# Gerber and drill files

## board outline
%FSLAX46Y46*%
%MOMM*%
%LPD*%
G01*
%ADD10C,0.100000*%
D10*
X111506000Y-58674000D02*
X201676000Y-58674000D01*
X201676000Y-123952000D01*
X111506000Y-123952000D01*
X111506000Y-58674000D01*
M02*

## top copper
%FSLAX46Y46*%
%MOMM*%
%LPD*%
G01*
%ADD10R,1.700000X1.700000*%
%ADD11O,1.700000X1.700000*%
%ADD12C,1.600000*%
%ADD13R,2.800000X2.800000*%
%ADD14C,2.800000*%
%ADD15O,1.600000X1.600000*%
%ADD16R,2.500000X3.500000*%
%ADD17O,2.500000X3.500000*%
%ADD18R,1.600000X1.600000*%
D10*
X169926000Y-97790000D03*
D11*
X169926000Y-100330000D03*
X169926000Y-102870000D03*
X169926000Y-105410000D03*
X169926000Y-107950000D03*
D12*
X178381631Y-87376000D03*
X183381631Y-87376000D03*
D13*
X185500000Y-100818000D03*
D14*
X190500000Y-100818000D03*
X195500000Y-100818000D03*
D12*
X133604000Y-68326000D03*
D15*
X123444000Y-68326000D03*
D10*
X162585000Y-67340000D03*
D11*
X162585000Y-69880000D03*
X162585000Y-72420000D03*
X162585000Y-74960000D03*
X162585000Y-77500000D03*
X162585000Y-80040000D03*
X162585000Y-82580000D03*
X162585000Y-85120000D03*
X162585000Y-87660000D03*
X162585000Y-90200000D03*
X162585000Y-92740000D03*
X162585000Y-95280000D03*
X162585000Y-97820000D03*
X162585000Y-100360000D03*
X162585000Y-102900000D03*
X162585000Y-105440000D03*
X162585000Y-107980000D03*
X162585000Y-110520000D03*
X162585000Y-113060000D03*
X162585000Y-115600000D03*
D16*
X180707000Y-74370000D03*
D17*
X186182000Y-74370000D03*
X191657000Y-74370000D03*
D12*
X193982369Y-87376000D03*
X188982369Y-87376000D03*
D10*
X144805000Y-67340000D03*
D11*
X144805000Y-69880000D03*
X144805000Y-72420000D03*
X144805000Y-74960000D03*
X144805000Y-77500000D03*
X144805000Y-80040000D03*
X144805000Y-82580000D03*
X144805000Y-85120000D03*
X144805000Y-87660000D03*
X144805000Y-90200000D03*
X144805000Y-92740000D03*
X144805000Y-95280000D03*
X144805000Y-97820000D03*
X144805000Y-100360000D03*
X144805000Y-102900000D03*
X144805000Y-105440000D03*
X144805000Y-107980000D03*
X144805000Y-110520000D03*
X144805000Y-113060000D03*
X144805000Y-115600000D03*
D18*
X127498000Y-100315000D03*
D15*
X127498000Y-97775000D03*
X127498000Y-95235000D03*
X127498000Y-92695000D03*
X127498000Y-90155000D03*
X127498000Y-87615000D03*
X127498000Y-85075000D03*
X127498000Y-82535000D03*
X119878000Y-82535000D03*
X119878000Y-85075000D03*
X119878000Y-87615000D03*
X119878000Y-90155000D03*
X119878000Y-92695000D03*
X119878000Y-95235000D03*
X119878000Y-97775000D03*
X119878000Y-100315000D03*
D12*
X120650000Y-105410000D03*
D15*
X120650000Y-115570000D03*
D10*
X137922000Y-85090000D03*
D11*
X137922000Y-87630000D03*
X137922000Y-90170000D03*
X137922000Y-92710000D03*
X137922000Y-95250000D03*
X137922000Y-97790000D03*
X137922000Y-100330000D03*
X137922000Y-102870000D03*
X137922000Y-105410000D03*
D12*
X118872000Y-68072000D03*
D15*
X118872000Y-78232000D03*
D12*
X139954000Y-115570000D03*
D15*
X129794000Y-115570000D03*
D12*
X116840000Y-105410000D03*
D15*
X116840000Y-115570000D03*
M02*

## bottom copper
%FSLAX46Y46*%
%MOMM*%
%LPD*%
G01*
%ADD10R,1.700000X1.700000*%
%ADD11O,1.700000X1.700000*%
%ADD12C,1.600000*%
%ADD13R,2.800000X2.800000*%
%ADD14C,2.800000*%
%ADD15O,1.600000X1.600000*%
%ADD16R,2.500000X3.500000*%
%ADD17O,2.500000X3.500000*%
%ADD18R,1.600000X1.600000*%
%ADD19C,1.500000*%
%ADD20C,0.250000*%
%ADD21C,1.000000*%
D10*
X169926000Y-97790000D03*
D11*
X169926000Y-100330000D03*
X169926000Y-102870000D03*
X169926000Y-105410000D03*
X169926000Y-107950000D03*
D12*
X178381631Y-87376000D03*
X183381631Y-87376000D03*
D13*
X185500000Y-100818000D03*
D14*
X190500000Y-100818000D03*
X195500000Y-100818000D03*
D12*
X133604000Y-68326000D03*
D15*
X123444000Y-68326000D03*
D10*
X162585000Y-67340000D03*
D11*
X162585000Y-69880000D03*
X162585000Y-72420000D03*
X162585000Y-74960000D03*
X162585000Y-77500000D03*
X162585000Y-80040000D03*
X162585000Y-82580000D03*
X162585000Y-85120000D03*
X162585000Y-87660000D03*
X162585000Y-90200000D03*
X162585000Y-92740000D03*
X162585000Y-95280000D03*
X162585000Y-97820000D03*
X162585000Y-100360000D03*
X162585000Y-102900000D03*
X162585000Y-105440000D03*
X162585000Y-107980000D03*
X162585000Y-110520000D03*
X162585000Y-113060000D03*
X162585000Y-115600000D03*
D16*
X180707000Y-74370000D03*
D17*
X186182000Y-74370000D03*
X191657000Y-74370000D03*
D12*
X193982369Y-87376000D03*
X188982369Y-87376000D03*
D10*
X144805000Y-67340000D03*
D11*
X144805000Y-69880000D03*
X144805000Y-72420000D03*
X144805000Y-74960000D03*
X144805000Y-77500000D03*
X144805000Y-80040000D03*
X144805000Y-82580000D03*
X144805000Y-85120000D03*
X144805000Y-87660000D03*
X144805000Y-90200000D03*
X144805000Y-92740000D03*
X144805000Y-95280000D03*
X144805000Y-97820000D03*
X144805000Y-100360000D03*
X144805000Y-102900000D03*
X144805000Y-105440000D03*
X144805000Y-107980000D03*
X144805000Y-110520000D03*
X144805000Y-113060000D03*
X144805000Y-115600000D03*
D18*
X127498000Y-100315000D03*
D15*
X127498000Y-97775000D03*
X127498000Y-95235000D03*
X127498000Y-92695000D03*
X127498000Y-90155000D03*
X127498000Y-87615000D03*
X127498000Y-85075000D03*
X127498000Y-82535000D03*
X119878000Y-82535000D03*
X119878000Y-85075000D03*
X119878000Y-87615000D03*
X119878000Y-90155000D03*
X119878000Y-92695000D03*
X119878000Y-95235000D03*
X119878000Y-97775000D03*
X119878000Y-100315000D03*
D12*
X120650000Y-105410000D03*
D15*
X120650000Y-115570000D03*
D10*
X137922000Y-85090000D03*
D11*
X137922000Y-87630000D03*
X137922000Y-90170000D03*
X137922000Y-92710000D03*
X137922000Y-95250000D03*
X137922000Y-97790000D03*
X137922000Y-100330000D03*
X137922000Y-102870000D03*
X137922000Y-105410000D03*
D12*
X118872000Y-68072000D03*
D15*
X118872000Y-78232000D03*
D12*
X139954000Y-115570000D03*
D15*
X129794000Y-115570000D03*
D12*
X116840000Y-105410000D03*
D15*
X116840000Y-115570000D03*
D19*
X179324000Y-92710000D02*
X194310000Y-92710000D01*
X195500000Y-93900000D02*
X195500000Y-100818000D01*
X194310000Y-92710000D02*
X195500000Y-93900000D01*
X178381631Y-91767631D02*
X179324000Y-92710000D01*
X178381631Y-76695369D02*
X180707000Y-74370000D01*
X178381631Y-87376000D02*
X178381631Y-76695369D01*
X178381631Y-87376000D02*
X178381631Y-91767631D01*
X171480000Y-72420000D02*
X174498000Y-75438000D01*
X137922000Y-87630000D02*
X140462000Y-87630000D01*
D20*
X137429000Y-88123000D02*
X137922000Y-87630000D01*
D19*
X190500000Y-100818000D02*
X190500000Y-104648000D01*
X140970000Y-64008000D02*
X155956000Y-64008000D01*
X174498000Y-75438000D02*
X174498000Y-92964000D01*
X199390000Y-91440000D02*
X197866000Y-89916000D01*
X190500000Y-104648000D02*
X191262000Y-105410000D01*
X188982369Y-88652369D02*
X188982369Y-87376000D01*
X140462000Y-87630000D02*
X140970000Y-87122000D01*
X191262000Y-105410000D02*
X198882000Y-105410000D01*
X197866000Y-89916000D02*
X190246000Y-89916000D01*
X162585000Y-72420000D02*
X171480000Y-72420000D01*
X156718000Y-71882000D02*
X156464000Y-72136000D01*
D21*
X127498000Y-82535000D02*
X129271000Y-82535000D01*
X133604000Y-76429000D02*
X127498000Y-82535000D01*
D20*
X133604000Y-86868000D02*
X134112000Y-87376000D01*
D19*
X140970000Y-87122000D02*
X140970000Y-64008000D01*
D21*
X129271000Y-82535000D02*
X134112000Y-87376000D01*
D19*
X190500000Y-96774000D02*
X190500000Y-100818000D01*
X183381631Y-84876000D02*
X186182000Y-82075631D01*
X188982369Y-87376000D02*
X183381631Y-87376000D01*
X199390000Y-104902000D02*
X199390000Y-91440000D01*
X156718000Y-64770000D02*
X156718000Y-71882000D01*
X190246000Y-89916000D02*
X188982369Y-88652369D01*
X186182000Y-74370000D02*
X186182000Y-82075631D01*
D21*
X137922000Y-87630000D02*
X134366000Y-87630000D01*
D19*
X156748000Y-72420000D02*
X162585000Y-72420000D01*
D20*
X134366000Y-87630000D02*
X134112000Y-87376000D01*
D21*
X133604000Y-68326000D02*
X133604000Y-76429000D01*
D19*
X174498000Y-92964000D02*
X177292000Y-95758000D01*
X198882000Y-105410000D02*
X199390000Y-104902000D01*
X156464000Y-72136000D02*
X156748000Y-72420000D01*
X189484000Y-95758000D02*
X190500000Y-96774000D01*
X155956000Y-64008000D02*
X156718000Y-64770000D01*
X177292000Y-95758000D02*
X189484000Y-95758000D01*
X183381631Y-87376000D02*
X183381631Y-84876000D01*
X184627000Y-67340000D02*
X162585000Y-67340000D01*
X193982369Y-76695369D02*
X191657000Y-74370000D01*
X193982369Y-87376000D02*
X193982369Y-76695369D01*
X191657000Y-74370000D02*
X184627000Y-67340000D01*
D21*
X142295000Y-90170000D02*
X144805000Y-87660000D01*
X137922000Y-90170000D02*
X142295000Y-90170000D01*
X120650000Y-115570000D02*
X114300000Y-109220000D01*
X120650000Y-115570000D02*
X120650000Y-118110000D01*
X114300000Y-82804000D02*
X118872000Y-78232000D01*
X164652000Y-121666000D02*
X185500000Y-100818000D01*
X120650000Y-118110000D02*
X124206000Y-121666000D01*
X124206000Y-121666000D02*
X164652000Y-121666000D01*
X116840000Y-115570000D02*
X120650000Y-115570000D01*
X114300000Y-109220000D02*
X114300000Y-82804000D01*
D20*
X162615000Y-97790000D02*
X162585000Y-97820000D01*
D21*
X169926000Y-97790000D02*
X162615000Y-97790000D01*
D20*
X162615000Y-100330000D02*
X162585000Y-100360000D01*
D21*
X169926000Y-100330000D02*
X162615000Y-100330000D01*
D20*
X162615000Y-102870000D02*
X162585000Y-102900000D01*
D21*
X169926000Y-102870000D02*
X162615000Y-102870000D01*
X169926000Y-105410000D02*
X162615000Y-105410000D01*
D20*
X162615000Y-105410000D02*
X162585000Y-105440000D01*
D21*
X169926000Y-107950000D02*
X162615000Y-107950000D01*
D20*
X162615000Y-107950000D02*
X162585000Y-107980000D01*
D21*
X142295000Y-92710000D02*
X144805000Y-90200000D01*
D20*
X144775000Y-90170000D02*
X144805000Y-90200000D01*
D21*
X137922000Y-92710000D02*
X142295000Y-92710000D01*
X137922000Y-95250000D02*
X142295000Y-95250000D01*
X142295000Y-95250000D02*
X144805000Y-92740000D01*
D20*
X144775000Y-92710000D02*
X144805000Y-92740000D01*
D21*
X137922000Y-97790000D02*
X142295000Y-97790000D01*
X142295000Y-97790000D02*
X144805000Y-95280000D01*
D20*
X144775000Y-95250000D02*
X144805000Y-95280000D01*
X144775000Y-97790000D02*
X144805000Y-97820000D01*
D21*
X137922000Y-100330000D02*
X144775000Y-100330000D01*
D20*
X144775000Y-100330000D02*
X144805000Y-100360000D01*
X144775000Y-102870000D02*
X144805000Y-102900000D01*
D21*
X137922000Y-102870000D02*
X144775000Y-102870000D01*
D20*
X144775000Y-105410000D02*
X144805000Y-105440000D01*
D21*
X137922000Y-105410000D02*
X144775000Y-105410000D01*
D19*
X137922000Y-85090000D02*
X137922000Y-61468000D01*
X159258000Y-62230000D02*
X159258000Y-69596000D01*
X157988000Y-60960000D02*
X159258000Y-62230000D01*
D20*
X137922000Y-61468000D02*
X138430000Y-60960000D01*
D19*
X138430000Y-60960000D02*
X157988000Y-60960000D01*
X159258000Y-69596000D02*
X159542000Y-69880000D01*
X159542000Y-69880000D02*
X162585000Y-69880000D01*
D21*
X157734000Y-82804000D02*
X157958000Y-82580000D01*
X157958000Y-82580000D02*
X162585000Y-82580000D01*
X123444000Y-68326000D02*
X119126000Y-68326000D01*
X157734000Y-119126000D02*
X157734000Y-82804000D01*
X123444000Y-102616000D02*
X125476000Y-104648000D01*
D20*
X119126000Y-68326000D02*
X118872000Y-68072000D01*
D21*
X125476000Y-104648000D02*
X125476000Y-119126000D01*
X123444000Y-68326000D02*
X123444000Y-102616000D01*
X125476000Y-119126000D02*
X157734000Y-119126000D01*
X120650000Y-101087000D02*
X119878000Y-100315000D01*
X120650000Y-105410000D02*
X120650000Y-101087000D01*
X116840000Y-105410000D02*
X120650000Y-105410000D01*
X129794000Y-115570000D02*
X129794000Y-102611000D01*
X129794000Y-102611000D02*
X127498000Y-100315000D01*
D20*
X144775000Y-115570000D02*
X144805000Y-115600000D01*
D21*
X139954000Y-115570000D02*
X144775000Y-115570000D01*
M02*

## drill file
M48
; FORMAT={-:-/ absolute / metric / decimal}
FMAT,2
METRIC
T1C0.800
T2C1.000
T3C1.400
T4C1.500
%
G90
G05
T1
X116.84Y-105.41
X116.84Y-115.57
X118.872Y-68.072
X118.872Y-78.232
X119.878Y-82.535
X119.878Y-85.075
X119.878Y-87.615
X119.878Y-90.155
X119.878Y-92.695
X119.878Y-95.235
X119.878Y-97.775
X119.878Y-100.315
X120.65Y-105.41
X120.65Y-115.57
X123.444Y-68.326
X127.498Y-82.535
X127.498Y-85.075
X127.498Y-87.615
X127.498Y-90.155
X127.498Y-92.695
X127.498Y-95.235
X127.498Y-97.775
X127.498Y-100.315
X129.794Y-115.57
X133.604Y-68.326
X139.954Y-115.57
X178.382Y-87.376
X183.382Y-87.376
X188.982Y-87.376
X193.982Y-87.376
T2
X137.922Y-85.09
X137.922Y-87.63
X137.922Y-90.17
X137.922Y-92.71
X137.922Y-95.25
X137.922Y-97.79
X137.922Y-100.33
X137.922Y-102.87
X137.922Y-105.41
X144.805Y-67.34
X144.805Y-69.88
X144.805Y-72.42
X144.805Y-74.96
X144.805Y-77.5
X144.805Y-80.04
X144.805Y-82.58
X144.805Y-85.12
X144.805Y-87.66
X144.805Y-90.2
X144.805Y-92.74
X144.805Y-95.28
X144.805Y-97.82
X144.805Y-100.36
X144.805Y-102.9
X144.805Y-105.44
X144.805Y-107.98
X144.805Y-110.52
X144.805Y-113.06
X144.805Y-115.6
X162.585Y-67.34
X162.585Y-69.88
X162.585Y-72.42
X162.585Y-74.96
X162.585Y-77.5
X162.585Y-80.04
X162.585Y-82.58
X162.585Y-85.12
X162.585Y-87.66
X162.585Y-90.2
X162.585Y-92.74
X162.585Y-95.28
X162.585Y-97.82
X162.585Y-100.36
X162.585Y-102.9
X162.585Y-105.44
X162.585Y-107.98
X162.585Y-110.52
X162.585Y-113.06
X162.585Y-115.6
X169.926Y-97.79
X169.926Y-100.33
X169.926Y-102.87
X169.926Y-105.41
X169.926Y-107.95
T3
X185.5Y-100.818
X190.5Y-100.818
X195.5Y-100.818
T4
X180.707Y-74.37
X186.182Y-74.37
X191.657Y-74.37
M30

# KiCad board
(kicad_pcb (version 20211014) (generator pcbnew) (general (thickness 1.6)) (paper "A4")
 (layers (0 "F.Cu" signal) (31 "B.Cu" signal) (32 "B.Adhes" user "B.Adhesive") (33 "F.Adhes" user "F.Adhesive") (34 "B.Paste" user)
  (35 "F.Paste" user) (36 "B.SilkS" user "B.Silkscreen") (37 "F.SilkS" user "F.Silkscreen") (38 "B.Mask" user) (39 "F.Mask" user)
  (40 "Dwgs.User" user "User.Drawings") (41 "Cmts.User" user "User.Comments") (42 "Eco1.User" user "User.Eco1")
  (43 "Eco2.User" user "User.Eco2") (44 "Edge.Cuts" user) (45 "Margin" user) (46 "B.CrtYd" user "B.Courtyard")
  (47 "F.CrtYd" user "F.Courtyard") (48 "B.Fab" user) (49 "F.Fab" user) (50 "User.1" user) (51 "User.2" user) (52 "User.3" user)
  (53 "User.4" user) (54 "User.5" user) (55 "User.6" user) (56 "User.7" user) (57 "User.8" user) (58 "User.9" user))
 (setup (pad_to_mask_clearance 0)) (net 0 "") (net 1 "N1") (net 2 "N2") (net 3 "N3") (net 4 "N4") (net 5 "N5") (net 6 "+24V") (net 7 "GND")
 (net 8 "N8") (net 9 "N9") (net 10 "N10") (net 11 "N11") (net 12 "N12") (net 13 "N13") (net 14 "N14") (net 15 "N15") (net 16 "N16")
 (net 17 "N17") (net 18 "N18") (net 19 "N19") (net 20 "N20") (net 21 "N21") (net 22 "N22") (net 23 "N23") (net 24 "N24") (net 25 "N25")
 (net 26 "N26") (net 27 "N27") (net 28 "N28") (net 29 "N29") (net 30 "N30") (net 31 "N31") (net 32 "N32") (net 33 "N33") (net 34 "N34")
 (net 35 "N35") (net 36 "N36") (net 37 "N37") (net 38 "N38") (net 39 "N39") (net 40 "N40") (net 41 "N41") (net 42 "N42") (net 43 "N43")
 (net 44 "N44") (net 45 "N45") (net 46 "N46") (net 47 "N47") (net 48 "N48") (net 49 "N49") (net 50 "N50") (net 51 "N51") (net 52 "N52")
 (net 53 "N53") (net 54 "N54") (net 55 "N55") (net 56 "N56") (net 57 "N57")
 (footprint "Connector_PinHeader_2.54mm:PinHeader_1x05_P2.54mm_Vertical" (layer "F.Cu") (at 169.926 97.79)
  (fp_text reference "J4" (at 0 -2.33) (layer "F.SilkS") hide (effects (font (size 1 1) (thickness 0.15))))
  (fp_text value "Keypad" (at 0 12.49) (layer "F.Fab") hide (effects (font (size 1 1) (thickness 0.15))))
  (pad "1" thru_hole rect (at 0 0) (size 1.7 1.7) (drill 1) (layers *.Cu *.Mask) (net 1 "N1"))
  (pad "2" thru_hole oval (at 0 2.54) (size 1.7 1.7) (drill 1) (layers *.Cu *.Mask) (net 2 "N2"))
  (pad "3" thru_hole oval (at 0 5.08) (size 1.7 1.7) (drill 1) (layers *.Cu *.Mask) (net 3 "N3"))
  (pad "4" thru_hole oval (at 0 7.62) (size 1.7 1.7) (drill 1) (layers *.Cu *.Mask) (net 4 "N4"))
  (pad "5" thru_hole oval (at 0 10.16) (size 1.7 1.7) (drill 1) (layers *.Cu *.Mask) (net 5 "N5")))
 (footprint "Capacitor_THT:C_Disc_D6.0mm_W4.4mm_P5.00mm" (layer "F.Cu") (at 178.381631 87.376)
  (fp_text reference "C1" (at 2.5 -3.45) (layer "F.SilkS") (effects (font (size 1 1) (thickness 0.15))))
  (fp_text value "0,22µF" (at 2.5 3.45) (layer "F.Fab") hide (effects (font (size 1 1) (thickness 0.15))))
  (pad "1" thru_hole circle (at 0 0) (size 1.6 1.6) (drill 0.8) (layers *.Cu *.Mask) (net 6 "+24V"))
  (pad "2" thru_hole circle (at 5 0) (size 1.6 1.6) (drill 0.8) (layers *.Cu *.Mask) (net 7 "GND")))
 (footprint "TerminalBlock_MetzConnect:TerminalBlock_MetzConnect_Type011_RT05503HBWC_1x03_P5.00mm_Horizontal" (layer "F.Cu")
  (at 185.5 100.818)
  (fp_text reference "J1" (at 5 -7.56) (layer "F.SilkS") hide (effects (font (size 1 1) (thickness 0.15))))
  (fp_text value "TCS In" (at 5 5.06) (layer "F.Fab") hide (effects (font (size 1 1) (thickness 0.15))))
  (pad "1" thru_hole rect (at 0 0) (size 2.8 2.8) (drill 1.4) (layers *.Cu *.Mask) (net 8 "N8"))
  (pad "2" thru_hole circle (at 5 0) (size 2.8 2.8) (drill 1.4) (layers *.Cu *.Mask) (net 7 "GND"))
  (pad "3" thru_hole circle (at 10 0) (size 2.8 2.8) (drill 1.4) (layers *.Cu *.Mask) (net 6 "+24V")))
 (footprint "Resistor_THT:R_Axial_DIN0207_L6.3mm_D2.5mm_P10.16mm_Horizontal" (layer "F.Cu") (at 133.604 68.326 180)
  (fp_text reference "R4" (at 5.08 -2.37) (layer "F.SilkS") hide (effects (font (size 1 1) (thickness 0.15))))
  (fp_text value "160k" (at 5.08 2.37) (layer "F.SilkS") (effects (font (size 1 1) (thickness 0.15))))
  (pad "1" thru_hole circle (at 0 0 180) (size 1.6 1.6) (drill 0.8) (layers *.Cu *.Mask) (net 7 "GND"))
  (pad "2" thru_hole oval (at 10.16 0 180) (size 1.6 1.6) (drill 0.8) (layers *.Cu *.Mask) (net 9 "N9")))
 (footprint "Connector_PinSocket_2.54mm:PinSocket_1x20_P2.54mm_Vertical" (layer "F.Cu") (at 162.585 67.34)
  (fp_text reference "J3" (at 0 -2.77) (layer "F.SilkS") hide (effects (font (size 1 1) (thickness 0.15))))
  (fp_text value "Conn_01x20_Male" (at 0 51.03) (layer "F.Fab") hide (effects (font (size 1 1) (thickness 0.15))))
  (pad "1" thru_hole rect (at 0 0) (size 1.7 1.7) (drill 1) (layers *.Cu *.Mask) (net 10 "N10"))
  (pad "2" thru_hole oval (at 0 2.54) (size 1.7 1.7) (drill 1) (layers *.Cu *.Mask) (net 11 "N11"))
  (pad "3" thru_hole oval (at 0 5.08) (size 1.7 1.7) (drill 1) (layers *.Cu *.Mask) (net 7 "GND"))
  (pad "4" thru_hole oval (at 0 7.62) (size 1.7 1.7) (drill 1) (layers *.Cu *.Mask) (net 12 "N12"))
  (pad "5" thru_hole oval (at 0 10.16) (size 1.7 1.7) (drill 1) (layers *.Cu *.Mask) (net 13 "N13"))
  (pad "6" thru_hole oval (at 0 12.7) (size 1.7 1.7) (drill 1) (layers *.Cu *.Mask) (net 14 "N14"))
  (pad "7" thru_hole oval (at 0 15.24) (size 1.7 1.7) (drill 1) (layers *.Cu *.Mask) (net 9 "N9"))
  (pad "8" thru_hole oval (at 0 17.78) (size 1.7 1.7) (drill 1) (layers *.Cu *.Mask) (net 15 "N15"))
  (pad "9" thru_hole oval (at 0 20.32) (size 1.7 1.7) (drill 1) (layers *.Cu *.Mask) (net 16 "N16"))
  (pad "10" thru_hole oval (at 0 22.86) (size 1.7 1.7) (drill 1) (layers *.Cu *.Mask) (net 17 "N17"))
  (pad "11" thru_hole oval (at 0 25.4) (size 1.7 1.7) (drill 1) (layers *.Cu *.Mask) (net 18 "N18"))
  (pad "12" thru_hole oval (at 0 27.94) (size 1.7 1.7) (drill 1) (layers *.Cu *.Mask) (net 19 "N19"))
  (pad "13" thru_hole oval (at 0 30.48) (size 1.7 1.7) (drill 1) (layers *.Cu *.Mask) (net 1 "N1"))
  (pad "14" thru_hole oval (at 0 33.02) (size 1.7 1.7) (drill 1) (layers *.Cu *.Mask) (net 2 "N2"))
  (pad "15" thru_hole oval (at 0 35.56) (size 1.7 1.7) (drill 1) (layers *.Cu *.Mask) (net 3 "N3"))
  (pad "16" thru_hole oval (at 0 38.1) (size 1.7 1.7) (drill 1) (layers *.Cu *.Mask) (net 4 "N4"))
  (pad "17" thru_hole oval (at 0 40.64) (size 1.7 1.7) (drill 1) (layers *.Cu *.Mask) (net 5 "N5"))
  (pad "18" thru_hole oval (at 0 43.18) (size 1.7 1.7) (drill 1) (layers *.Cu *.Mask) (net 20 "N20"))
  (pad "19" thru_hole oval (at 0 45.72) (size 1.7 1.7) (drill 1) (layers *.Cu *.Mask) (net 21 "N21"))
  (pad "20" thru_hole oval (at 0 48.26) (size 1.7 1.7) (drill 1) (layers *.Cu *.Mask) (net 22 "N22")))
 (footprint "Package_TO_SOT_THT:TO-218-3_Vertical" (layer "F.Cu") (at 180.707 74.37)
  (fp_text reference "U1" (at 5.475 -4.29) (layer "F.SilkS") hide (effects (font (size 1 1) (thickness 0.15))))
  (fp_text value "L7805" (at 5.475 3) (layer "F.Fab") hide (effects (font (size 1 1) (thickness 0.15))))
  (pad "1" thru_hole rect (at 0 0) (size 2.5 3.5) (drill 1.5) (layers *.Cu *.Mask) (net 6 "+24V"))
  (pad "2" thru_hole oval (at 5.475 0) (size 2.5 3.5) (drill 1.5) (layers *.Cu *.Mask) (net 7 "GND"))
  (pad "3" thru_hole oval (at 10.95 0) (size 2.5 3.5) (drill 1.5) (layers *.Cu *.Mask) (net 10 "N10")))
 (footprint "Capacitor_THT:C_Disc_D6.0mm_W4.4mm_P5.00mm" (layer "F.Cu") (at 193.982369 87.376 180)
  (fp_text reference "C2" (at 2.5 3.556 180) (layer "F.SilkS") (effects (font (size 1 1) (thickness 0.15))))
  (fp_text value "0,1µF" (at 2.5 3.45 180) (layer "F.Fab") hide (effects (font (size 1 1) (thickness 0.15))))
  (pad "1" thru_hole circle (at 0 0 180) (size 1.6 1.6) (drill 0.8) (layers *.Cu *.Mask) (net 10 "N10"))
  (pad "2" thru_hole circle (at 5 0 180) (size 1.6 1.6) (drill 0.8) (layers *.Cu *.Mask) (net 7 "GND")))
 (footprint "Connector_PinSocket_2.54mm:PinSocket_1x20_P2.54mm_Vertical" (layer "F.Cu") (at 144.805 67.34)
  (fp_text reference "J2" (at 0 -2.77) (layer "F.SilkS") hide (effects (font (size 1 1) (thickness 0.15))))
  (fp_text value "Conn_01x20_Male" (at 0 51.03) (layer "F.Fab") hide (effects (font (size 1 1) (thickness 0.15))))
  (pad "1" thru_hole rect (at 0 0) (size 1.7 1.7) (drill 1) (layers *.Cu *.Mask) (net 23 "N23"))
  (pad "2" thru_hole oval (at 0 2.54) (size 1.7 1.7) (drill 1) (layers *.Cu *.Mask) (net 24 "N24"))
  (pad "3" thru_hole oval (at 0 5.08) (size 1.7 1.7) (drill 1) (layers *.Cu *.Mask) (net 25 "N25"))
  (pad "4" thru_hole oval (at 0 7.62) (size 1.7 1.7) (drill 1) (layers *.Cu *.Mask) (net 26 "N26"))
  (pad "5" thru_hole oval (at 0 10.16) (size 1.7 1.7) (drill 1) (layers *.Cu *.Mask) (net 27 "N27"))
  (pad "6" thru_hole oval (at 0 12.7) (size 1.7 1.7) (drill 1) (layers *.Cu *.Mask) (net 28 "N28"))
  (pad "7" thru_hole oval (at 0 15.24) (size 1.7 1.7) (drill 1) (layers *.Cu *.Mask) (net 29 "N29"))
  (pad "8" thru_hole oval (at 0 17.78) (size 1.7 1.7) (drill 1) (layers *.Cu *.Mask) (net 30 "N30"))
  (pad "9" thru_hole oval (at 0 20.32) (size 1.7 1.7) (drill 1) (layers *.Cu *.Mask) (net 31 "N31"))
  (pad "10" thru_hole oval (at 0 22.86) (size 1.7 1.7) (drill 1) (layers *.Cu *.Mask) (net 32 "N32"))
  (pad "11" thru_hole oval (at 0 25.4) (size 1.7 1.7) (drill 1) (layers *.Cu *.Mask) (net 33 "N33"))
  (pad "12" thru_hole oval (at 0 27.94) (size 1.7 1.7) (drill 1) (layers *.Cu *.Mask) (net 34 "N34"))
  (pad "13" thru_hole oval (at 0 30.48) (size 1.7 1.7) (drill 1) (layers *.Cu *.Mask) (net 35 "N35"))
  (pad "14" thru_hole oval (at 0 33.02) (size 1.7 1.7) (drill 1) (layers *.Cu *.Mask) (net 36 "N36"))
  (pad "15" thru_hole oval (at 0 35.56) (size 1.7 1.7) (drill 1) (layers *.Cu *.Mask) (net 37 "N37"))
  (pad "16" thru_hole oval (at 0 38.1) (size 1.7 1.7) (drill 1) (layers *.Cu *.Mask) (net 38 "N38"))
  (pad "17" thru_hole oval (at 0 40.64) (size 1.7 1.7) (drill 1) (layers *.Cu *.Mask) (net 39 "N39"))
  (pad "18" thru_hole oval (at 0 43.18) (size 1.7 1.7) (drill 1) (layers *.Cu *.Mask) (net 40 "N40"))
  (pad "19" thru_hole oval (at 0 45.72) (size 1.7 1.7) (drill 1) (layers *.Cu *.Mask) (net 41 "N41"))
  (pad "20" thru_hole oval (at 0 48.26) (size 1.7 1.7) (drill 1) (layers *.Cu *.Mask) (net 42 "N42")))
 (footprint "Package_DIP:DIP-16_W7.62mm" (layer "F.Cu") (at 127.498 100.315 180)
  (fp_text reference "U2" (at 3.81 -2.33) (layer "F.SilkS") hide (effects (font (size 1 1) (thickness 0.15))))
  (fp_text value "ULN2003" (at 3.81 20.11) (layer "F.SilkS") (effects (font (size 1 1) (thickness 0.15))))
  (pad "1" thru_hole rect (at 0 0 180) (size 1.6 1.6) (drill 0.8) (layers *.Cu *.Mask) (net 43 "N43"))
  (pad "2" thru_hole oval (at 0 2.54 180) (size 1.6 1.6) (drill 0.8) (layers *.Cu *.Mask) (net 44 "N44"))
  (pad "3" thru_hole oval (at 0 5.08 180) (size 1.6 1.6) (drill 0.8) (layers *.Cu *.Mask) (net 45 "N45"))
  (pad "4" thru_hole oval (at 0 7.62 180) (size 1.6 1.6) (drill 0.8) (layers *.Cu *.Mask) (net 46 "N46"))
  (pad "5" thru_hole oval (at 0 10.16 180) (size 1.6 1.6) (drill 0.8) (layers *.Cu *.Mask) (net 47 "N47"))
  (pad "6" thru_hole oval (at 0 12.7 180) (size 1.6 1.6) (drill 0.8) (layers *.Cu *.Mask) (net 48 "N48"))
  (pad "7" thru_hole oval (at 0 15.24 180) (size 1.6 1.6) (drill 0.8) (layers *.Cu *.Mask) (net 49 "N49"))
  (pad "8" thru_hole oval (at 0 17.78 180) (size 1.6 1.6) (drill 0.8) (layers *.Cu *.Mask) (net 7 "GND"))
  (pad "9" thru_hole oval (at 7.62 17.78 180) (size 1.6 1.6) (drill 0.8) (layers *.Cu *.Mask) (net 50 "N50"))
  (pad "10" thru_hole oval (at 7.62 15.24 180) (size 1.6 1.6) (drill 0.8) (layers *.Cu *.Mask) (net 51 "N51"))
  (pad "11" thru_hole oval (at 7.62 12.7 180) (size 1.6 1.6) (drill 0.8) (layers *.Cu *.Mask) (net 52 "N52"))
  (pad "12" thru_hole oval (at 7.62 10.16 180) (size 1.6 1.6) (drill 0.8) (layers *.Cu *.Mask) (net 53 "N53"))
  (pad "13" thru_hole oval (at 7.62 7.62 180) (size 1.6 1.6) (drill 0.8) (layers *.Cu *.Mask) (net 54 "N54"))
  (pad "14" thru_hole oval (at 7.62 5.08 180) (size 1.6 1.6) (drill 0.8) (layers *.Cu *.Mask) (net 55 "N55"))
  (pad "15" thru_hole oval (at 7.62 2.54 180) (size 1.6 1.6) (drill 0.8) (layers *.Cu *.Mask) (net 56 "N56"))
  (pad "16" thru_hole oval (at 7.62 0 180) (size 1.6 1.6) (drill 0.8) (layers *.Cu *.Mask) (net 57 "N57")))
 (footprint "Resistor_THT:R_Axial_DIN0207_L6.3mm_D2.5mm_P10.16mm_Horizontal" (layer "F.Cu") (at 120.65 105.41 -90)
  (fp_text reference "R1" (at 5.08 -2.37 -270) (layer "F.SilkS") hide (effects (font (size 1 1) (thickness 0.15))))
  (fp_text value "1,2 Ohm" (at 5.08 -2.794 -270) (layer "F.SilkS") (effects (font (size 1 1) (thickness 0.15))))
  (pad "1" thru_hole circle (at 0 0 270) (size 1.6 1.6) (drill 0.8) (layers *.Cu *.Mask) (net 57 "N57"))
  (pad "2" thru_hole oval (at 10.16 0 270) (size 1.6 1.6) (drill 0.8) (layers *.Cu *.Mask) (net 8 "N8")))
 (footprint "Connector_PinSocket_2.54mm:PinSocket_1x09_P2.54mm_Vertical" (layer "F.Cu") (at 137.922 85.09)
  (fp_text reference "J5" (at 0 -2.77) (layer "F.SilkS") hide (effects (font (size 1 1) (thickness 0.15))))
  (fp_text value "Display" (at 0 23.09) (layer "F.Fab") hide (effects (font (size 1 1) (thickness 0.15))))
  (pad "1" thru_hole rect (at 0 0) (size 1.7 1.7) (drill 1) (layers *.Cu *.Mask) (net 11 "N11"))
  (pad "2" thru_hole oval (at 0 2.54) (size 1.7 1.7) (drill 1) (layers *.Cu *.Mask) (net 7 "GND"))
  (pad "3" thru_hole oval (at 0 5.08) (size 1.7 1.7) (drill 1) (layers *.Cu *.Mask) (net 31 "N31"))
  (pad "4" thru_hole oval (at 0 7.62) (size 1.7 1.7) (drill 1) (layers *.Cu *.Mask) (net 32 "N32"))
  (pad "5" thru_hole oval (at 0 10.16) (size 1.7 1.7) (drill 1) (layers *.Cu *.Mask) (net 33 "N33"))
  (pad "6" thru_hole oval (at 0 12.7) (size 1.7 1.7) (drill 1) (layers *.Cu *.Mask) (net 34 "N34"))
  (pad "7" thru_hole oval (at 0 15.24) (size 1.7 1.7) (drill 1) (layers *.Cu *.Mask) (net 36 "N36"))
  (pad "8" thru_hole oval (at 0 17.78) (size 1.7 1.7) (drill 1) (layers *.Cu *.Mask) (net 37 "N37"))
  (pad "9" thru_hole oval (at 0 20.32) (size 1.7 1.7) (drill 1) (layers *.Cu *.Mask) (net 38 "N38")))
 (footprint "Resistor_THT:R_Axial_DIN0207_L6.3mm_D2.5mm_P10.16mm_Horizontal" (layer "F.Cu") (at 118.872 68.072 -90)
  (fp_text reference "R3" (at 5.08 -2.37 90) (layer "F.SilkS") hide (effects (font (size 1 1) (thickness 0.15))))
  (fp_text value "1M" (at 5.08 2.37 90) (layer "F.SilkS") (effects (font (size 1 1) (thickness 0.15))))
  (pad "1" thru_hole circle (at 0 0 270) (size 1.6 1.6) (drill 0.8) (layers *.Cu *.Mask) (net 9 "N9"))
  (pad "2" thru_hole oval (at 10.16 0 270) (size 1.6 1.6) (drill 0.8) (layers *.Cu *.Mask) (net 8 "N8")))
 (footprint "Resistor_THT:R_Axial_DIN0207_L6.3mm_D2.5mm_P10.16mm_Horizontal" (layer "F.Cu") (at 139.954 115.57 180)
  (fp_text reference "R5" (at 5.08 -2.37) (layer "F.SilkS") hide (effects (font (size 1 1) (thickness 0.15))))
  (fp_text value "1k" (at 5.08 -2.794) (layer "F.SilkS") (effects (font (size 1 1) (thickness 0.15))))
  (pad "1" thru_hole circle (at 0 0 180) (size 1.6 1.6) (drill 0.8) (layers *.Cu *.Mask) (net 42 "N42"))
  (pad "2" thru_hole oval (at 10.16 0 180) (size 1.6 1.6) (drill 0.8) (layers *.Cu *.Mask) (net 43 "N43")))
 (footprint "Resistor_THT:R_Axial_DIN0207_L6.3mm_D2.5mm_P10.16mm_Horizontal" (layer "F.Cu") (at 116.84 105.41 -90)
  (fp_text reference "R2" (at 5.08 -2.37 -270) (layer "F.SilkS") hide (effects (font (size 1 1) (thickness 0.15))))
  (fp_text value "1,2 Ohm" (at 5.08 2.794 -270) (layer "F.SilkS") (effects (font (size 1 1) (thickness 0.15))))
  (pad "1" thru_hole circle (at 0 0 270) (size 1.6 1.6) (drill 0.8) (layers *.Cu *.Mask) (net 57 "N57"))
  (pad "2" thru_hole oval (at 10.16 0 270) (size 1.6 1.6) (drill 0.8) (layers *.Cu *.Mask) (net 8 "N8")))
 (gr_rect (start 111.506 58.674) (end 201.676 123.952) (layer "Edge.Cuts") (width 0.1) (fill none))
 (segment (start 179.324 92.71) (end 194.31 92.71) (width 1.5) (layer "B.Cu") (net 6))
 (segment (start 195.5 93.9) (end 195.5 100.818) (width 1.5) (layer "B.Cu") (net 6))
 (segment (start 194.31 92.71) (end 195.5 93.9) (width 1.5) (layer "B.Cu") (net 6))
 (segment (start 178.381631 91.767631) (end 179.324 92.71) (width 1.5) (layer "B.Cu") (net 6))
 (segment (start 178.381631 76.695369) (end 180.707 74.37) (width 1.5) (layer "B.Cu") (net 6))
 (segment (start 178.381631 87.376) (end 178.381631 76.695369) (width 1.5) (layer "B.Cu") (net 6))
 (segment (start 178.381631 87.376) (end 178.381631 91.767631) (width 1.5) (layer "B.Cu") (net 6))
 (segment (start 171.48 72.42) (end 174.498 75.438) (width 1.5) (layer "B.Cu") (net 7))
 (segment (start 137.922 87.63) (end 140.462 87.63) (width 1.5) (layer "B.Cu") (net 7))
 (segment (start 137.429 88.123) (end 137.922 87.63) (width 0.25) (layer "B.Cu") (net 7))
 (segment (start 190.5 100.818) (end 190.5 104.648) (width 1.5) (layer "B.Cu") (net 7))
 (segment (start 140.97 64.008) (end 155.956 64.008) (width 1.5) (layer "B.Cu") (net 7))
 (segment (start 174.498 75.438) (end 174.498 92.964) (width 1.5) (layer "B.Cu") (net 7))
 (segment (start 199.39 91.44) (end 197.866 89.916) (width 1.5) (layer "B.Cu") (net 7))
 (segment (start 190.5 104.648) (end 191.262 105.41) (width 1.5) (layer "B.Cu") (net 7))
 (segment (start 188.982369 88.652369) (end 188.982369 87.376) (width 1.5) (layer "B.Cu") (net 7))
 (segment (start 140.462 87.63) (end 140.97 87.122) (width 1.5) (layer "B.Cu") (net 7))
 (segment (start 191.262 105.41) (end 198.882 105.41) (width 1.5) (layer "B.Cu") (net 7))
 (segment (start 197.866 89.916) (end 190.246 89.916) (width 1.5) (layer "B.Cu") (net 7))
 (segment (start 162.585 72.42) (end 171.48 72.42) (width 1.5) (layer "B.Cu") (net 7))
 (segment (start 156.718 71.882) (end 156.464 72.136) (width 1.5) (layer "B.Cu") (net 7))
 (segment (start 127.498 82.535) (end 129.271 82.535) (width 1) (layer "B.Cu") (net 7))
 (segment (start 133.604 76.429) (end 127.498 82.535) (width 1) (layer "B.Cu") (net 7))
 (segment (start 133.604 86.868) (end 134.112 87.376) (width 0.25) (layer "B.Cu") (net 7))
 (segment (start 140.97 87.122) (end 140.97 64.008) (width 1.5) (layer "B.Cu") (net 7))
 (segment (start 129.271 82.535) (end 134.112 87.376) (width 1) (layer "B.Cu") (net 7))
 (segment (start 190.5 96.774) (end 190.5 100.818) (width 1.5) (layer "B.Cu") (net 7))
 (segment (start 183.381631 84.876) (end 186.182 82.075631) (width 1.5) (layer "B.Cu") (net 7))
 (segment (start 188.982369 87.376) (end 183.381631 87.376) (width 1.5) (layer "B.Cu") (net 7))
 (segment (start 199.39 104.902) (end 199.39 91.44) (width 1.5) (layer "B.Cu") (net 7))
 (segment (start 156.718 64.77) (end 156.718 71.882) (width 1.5) (layer "B.Cu") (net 7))
 (segment (start 190.246 89.916) (end 188.982369 88.652369) (width 1.5) (layer "B.Cu") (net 7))
 (segment (start 186.182 74.37) (end 186.182 82.075631) (width 1.5) (layer "B.Cu") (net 7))
 (segment (start 137.922 87.63) (end 134.366 87.63) (width 1) (layer "B.Cu") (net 7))
 (segment (start 156.748 72.42) (end 162.585 72.42) (width 1.5) (layer "B.Cu") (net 7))
 (segment (start 134.366 87.63) (end 134.112 87.376) (width 0.25) (layer "B.Cu") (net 7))
 (segment (start 133.604 68.326) (end 133.604 76.429) (width 1) (layer "B.Cu") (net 7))
 (segment (start 174.498 92.964) (end 177.292 95.758) (width 1.5) (layer "B.Cu") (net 7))
 (segment (start 198.882 105.41) (end 199.39 104.902) (width 1.5) (layer "B.Cu") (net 7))
 (segment (start 156.464 72.136) (end 156.748 72.42) (width 1.5) (layer "B.Cu") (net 7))
 (segment (start 189.484 95.758) (end 190.5 96.774) (width 1.5) (layer "B.Cu") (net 7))
 (segment (start 155.956 64.008) (end 156.718 64.77) (width 1.5) (layer "B.Cu") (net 7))
 (segment (start 177.292 95.758) (end 189.484 95.758) (width 1.5) (layer "B.Cu") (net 7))
 (segment (start 183.381631 87.376) (end 183.381631 84.876) (width 1.5) (layer "B.Cu") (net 7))
 (segment (start 184.627 67.34) (end 162.585 67.34) (width 1.5) (layer "B.Cu") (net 10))
 (segment (start 193.982369 76.695369) (end 191.657 74.37) (width 1.5) (layer "B.Cu") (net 10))
 (segment (start 193.982369 87.376) (end 193.982369 76.695369) (width 1.5) (layer "B.Cu") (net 10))
 (segment (start 191.657 74.37) (end 184.627 67.34) (width 1.5) (layer "B.Cu") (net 10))
 (segment (start 142.295 90.17) (end 144.805 87.66) (width 1) (layer "B.Cu") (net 31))
 (segment (start 137.922 90.17) (end 142.295 90.17) (width 1) (layer "B.Cu") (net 31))
 (segment (start 120.65 115.57) (end 114.3 109.22) (width 1) (layer "B.Cu") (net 8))
 (segment (start 120.65 115.57) (end 120.65 118.11) (width 1) (layer "B.Cu") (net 8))
 (segment (start 114.3 82.804) (end 118.872 78.232) (width 1) (layer "B.Cu") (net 8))
 (segment (start 164.652 121.666) (end 185.5 100.818) (width 1) (layer "B.Cu") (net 8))
 (segment (start 120.65 118.11) (end 124.206 121.666) (width 1) (layer "B.Cu") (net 8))
 (segment (start 124.206 121.666) (end 164.652 121.666) (width 1) (layer "B.Cu") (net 8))
 (segment (start 116.84 115.57) (end 120.65 115.57) (width 1) (layer "B.Cu") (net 8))
 (segment (start 114.3 109.22) (end 114.3 82.804) (width 1) (layer "B.Cu") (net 8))
 (segment (start 162.615 97.79) (end 162.585 97.82) (width 0.25) (layer "B.Cu") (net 1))
 (segment (start 169.926 97.79) (end 162.615 97.79) (width 1) (layer "B.Cu") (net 1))
 (segment (start 162.615 100.33) (end 162.585 100.36) (width 0.25) (layer "B.Cu") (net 2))
 (segment (start 169.926 100.33) (end 162.615 100.33) (width 1) (layer "B.Cu") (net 2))
 (segment (start 162.615 102.87) (end 162.585 102.9) (width 0.25) (layer "B.Cu") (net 3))
 (segment (start 169.926 102.87) (end 162.615 102.87) (width 1) (layer "B.Cu") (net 3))
 (segment (start 169.926 105.41) (end 162.615 105.41) (width 1) (layer "B.Cu") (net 4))
 (segment (start 162.615 105.41) (end 162.585 105.44) (width 0.25) (layer "B.Cu") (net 4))
 (segment (start 169.926 107.95) (end 162.615 107.95) (width 1) (layer "B.Cu") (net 5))
 (segment (start 162.615 107.95) (end 162.585 107.98) (width 0.25) (layer "B.Cu") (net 5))
 (segment (start 142.295 92.71) (end 144.805 90.2) (width 1) (layer "B.Cu") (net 32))
 (segment (start 144.775 90.17) (end 144.805 90.2) (width 0.25) (layer "B.Cu") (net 32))
 (segment (start 137.922 92.71) (end 142.295 92.71) (width 1) (layer "B.Cu") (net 32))
 (segment (start 137.922 95.25) (end 142.295 95.25) (width 1) (layer "B.Cu") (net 33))
 (segment (start 142.295 95.25) (end 144.805 92.74) (width 1) (layer "B.Cu") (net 33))
 (segment (start 144.775 92.71) (end 144.805 92.74) (width 0.25) (layer "B.Cu") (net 33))
 (segment (start 137.922 97.79) (end 142.295 97.79) (width 1) (layer "B.Cu") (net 34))
 (segment (start 142.295 97.79) (end 144.805 95.28) (width 1) (layer "B.Cu") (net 34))
 (segment (start 144.775 95.25) (end 144.805 95.28) (width 0.25) (layer "B.Cu") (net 34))
 (segment (start 144.775 97.79) (end 144.805 97.82) (width 0.25) (layer "B.Cu") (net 35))
 (segment (start 137.922 100.33) (end 144.775 100.33) (width 1) (layer "B.Cu") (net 36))
 (segment (start 144.775 100.33) (end 144.805 100.36) (width 0.25) (layer "B.Cu") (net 36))
 (segment (start 144.775 102.87) (end 144.805 102.9) (width 0.25) (layer "B.Cu") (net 37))
 (segment (start 137.922 102.87) (end 144.775 102.87) (width 1) (layer "B.Cu") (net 37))
 (segment (start 144.775 105.41) (end 144.805 105.44) (width 0.25) (layer "B.Cu") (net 38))
 (segment (start 137.922 105.41) (end 144.775 105.41) (width 1) (layer "B.Cu") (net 38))
 (segment (start 137.922 85.09) (end 137.922 61.468) (width 1.5) (layer "B.Cu") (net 11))
 (segment (start 159.258 62.23) (end 159.258 69.596) (width 1.5) (layer "B.Cu") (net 11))
 (segment (start 157.988 60.96) (end 159.258 62.23) (width 1.5) (layer "B.Cu") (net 11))
 (segment (start 137.922 61.468) (end 138.43 60.96) (width 0.25) (layer "B.Cu") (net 11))
 (segment (start 138.43 60.96) (end 157.988 60.96) (width 1.5) (layer "B.Cu") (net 11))
 (segment (start 159.258 69.596) (end 159.542 69.88) (width 1.5) (layer "B.Cu") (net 11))
 (segment (start 159.542 69.88) (end 162.585 69.88) (width 1.5) (layer "B.Cu") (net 11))
 (segment (start 157.734 82.804) (end 157.958 82.58) (width 1) (layer "B.Cu") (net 9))
 (segment (start 157.958 82.58) (end 162.585 82.58) (width 1) (layer "B.Cu") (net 9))
 (segment (start 123.444 68.326) (end 119.126 68.326) (width 1) (layer "B.Cu") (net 9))
 (segment (start 157.734 119.126) (end 157.734 82.804) (width 1) (layer "B.Cu") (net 9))
 (segment (start 123.444 102.616) (end 125.476 104.648) (width 1) (layer "B.Cu") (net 9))
 (segment (start 119.126 68.326) (end 118.872 68.072) (width 0.25) (layer "B.Cu") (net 9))
 (segment (start 125.476 104.648) (end 125.476 119.126) (width 1) (layer "B.Cu") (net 9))
 (segment (start 123.444 68.326) (end 123.444 102.616) (width 1) (layer "B.Cu") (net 9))
 (segment (start 125.476 119.126) (end 157.734 119.126) (width 1) (layer "B.Cu") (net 9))
 (segment (start 120.65 101.087) (end 119.878 100.315) (width 1) (layer "B.Cu") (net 57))
 (segment (start 120.65 105.41) (end 120.65 101.087) (width 1) (layer "B.Cu") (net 57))
 (segment (start 116.84 105.41) (end 120.65 105.41) (width 1) (layer "B.Cu") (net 57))
 (segment (start 129.794 115.57) (end 129.794 102.611) (width 1) (layer "B.Cu") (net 43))
 (segment (start 129.794 102.611) (end 127.498 100.315) (width 1) (layer "B.Cu") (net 43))
 (segment (start 144.775 115.57) (end 144.805 115.6) (width 0.25) (layer "B.Cu") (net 42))
 (segment (start 139.954 115.57) (end 144.775 115.57) (width 1) (layer "B.Cu") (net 42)))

